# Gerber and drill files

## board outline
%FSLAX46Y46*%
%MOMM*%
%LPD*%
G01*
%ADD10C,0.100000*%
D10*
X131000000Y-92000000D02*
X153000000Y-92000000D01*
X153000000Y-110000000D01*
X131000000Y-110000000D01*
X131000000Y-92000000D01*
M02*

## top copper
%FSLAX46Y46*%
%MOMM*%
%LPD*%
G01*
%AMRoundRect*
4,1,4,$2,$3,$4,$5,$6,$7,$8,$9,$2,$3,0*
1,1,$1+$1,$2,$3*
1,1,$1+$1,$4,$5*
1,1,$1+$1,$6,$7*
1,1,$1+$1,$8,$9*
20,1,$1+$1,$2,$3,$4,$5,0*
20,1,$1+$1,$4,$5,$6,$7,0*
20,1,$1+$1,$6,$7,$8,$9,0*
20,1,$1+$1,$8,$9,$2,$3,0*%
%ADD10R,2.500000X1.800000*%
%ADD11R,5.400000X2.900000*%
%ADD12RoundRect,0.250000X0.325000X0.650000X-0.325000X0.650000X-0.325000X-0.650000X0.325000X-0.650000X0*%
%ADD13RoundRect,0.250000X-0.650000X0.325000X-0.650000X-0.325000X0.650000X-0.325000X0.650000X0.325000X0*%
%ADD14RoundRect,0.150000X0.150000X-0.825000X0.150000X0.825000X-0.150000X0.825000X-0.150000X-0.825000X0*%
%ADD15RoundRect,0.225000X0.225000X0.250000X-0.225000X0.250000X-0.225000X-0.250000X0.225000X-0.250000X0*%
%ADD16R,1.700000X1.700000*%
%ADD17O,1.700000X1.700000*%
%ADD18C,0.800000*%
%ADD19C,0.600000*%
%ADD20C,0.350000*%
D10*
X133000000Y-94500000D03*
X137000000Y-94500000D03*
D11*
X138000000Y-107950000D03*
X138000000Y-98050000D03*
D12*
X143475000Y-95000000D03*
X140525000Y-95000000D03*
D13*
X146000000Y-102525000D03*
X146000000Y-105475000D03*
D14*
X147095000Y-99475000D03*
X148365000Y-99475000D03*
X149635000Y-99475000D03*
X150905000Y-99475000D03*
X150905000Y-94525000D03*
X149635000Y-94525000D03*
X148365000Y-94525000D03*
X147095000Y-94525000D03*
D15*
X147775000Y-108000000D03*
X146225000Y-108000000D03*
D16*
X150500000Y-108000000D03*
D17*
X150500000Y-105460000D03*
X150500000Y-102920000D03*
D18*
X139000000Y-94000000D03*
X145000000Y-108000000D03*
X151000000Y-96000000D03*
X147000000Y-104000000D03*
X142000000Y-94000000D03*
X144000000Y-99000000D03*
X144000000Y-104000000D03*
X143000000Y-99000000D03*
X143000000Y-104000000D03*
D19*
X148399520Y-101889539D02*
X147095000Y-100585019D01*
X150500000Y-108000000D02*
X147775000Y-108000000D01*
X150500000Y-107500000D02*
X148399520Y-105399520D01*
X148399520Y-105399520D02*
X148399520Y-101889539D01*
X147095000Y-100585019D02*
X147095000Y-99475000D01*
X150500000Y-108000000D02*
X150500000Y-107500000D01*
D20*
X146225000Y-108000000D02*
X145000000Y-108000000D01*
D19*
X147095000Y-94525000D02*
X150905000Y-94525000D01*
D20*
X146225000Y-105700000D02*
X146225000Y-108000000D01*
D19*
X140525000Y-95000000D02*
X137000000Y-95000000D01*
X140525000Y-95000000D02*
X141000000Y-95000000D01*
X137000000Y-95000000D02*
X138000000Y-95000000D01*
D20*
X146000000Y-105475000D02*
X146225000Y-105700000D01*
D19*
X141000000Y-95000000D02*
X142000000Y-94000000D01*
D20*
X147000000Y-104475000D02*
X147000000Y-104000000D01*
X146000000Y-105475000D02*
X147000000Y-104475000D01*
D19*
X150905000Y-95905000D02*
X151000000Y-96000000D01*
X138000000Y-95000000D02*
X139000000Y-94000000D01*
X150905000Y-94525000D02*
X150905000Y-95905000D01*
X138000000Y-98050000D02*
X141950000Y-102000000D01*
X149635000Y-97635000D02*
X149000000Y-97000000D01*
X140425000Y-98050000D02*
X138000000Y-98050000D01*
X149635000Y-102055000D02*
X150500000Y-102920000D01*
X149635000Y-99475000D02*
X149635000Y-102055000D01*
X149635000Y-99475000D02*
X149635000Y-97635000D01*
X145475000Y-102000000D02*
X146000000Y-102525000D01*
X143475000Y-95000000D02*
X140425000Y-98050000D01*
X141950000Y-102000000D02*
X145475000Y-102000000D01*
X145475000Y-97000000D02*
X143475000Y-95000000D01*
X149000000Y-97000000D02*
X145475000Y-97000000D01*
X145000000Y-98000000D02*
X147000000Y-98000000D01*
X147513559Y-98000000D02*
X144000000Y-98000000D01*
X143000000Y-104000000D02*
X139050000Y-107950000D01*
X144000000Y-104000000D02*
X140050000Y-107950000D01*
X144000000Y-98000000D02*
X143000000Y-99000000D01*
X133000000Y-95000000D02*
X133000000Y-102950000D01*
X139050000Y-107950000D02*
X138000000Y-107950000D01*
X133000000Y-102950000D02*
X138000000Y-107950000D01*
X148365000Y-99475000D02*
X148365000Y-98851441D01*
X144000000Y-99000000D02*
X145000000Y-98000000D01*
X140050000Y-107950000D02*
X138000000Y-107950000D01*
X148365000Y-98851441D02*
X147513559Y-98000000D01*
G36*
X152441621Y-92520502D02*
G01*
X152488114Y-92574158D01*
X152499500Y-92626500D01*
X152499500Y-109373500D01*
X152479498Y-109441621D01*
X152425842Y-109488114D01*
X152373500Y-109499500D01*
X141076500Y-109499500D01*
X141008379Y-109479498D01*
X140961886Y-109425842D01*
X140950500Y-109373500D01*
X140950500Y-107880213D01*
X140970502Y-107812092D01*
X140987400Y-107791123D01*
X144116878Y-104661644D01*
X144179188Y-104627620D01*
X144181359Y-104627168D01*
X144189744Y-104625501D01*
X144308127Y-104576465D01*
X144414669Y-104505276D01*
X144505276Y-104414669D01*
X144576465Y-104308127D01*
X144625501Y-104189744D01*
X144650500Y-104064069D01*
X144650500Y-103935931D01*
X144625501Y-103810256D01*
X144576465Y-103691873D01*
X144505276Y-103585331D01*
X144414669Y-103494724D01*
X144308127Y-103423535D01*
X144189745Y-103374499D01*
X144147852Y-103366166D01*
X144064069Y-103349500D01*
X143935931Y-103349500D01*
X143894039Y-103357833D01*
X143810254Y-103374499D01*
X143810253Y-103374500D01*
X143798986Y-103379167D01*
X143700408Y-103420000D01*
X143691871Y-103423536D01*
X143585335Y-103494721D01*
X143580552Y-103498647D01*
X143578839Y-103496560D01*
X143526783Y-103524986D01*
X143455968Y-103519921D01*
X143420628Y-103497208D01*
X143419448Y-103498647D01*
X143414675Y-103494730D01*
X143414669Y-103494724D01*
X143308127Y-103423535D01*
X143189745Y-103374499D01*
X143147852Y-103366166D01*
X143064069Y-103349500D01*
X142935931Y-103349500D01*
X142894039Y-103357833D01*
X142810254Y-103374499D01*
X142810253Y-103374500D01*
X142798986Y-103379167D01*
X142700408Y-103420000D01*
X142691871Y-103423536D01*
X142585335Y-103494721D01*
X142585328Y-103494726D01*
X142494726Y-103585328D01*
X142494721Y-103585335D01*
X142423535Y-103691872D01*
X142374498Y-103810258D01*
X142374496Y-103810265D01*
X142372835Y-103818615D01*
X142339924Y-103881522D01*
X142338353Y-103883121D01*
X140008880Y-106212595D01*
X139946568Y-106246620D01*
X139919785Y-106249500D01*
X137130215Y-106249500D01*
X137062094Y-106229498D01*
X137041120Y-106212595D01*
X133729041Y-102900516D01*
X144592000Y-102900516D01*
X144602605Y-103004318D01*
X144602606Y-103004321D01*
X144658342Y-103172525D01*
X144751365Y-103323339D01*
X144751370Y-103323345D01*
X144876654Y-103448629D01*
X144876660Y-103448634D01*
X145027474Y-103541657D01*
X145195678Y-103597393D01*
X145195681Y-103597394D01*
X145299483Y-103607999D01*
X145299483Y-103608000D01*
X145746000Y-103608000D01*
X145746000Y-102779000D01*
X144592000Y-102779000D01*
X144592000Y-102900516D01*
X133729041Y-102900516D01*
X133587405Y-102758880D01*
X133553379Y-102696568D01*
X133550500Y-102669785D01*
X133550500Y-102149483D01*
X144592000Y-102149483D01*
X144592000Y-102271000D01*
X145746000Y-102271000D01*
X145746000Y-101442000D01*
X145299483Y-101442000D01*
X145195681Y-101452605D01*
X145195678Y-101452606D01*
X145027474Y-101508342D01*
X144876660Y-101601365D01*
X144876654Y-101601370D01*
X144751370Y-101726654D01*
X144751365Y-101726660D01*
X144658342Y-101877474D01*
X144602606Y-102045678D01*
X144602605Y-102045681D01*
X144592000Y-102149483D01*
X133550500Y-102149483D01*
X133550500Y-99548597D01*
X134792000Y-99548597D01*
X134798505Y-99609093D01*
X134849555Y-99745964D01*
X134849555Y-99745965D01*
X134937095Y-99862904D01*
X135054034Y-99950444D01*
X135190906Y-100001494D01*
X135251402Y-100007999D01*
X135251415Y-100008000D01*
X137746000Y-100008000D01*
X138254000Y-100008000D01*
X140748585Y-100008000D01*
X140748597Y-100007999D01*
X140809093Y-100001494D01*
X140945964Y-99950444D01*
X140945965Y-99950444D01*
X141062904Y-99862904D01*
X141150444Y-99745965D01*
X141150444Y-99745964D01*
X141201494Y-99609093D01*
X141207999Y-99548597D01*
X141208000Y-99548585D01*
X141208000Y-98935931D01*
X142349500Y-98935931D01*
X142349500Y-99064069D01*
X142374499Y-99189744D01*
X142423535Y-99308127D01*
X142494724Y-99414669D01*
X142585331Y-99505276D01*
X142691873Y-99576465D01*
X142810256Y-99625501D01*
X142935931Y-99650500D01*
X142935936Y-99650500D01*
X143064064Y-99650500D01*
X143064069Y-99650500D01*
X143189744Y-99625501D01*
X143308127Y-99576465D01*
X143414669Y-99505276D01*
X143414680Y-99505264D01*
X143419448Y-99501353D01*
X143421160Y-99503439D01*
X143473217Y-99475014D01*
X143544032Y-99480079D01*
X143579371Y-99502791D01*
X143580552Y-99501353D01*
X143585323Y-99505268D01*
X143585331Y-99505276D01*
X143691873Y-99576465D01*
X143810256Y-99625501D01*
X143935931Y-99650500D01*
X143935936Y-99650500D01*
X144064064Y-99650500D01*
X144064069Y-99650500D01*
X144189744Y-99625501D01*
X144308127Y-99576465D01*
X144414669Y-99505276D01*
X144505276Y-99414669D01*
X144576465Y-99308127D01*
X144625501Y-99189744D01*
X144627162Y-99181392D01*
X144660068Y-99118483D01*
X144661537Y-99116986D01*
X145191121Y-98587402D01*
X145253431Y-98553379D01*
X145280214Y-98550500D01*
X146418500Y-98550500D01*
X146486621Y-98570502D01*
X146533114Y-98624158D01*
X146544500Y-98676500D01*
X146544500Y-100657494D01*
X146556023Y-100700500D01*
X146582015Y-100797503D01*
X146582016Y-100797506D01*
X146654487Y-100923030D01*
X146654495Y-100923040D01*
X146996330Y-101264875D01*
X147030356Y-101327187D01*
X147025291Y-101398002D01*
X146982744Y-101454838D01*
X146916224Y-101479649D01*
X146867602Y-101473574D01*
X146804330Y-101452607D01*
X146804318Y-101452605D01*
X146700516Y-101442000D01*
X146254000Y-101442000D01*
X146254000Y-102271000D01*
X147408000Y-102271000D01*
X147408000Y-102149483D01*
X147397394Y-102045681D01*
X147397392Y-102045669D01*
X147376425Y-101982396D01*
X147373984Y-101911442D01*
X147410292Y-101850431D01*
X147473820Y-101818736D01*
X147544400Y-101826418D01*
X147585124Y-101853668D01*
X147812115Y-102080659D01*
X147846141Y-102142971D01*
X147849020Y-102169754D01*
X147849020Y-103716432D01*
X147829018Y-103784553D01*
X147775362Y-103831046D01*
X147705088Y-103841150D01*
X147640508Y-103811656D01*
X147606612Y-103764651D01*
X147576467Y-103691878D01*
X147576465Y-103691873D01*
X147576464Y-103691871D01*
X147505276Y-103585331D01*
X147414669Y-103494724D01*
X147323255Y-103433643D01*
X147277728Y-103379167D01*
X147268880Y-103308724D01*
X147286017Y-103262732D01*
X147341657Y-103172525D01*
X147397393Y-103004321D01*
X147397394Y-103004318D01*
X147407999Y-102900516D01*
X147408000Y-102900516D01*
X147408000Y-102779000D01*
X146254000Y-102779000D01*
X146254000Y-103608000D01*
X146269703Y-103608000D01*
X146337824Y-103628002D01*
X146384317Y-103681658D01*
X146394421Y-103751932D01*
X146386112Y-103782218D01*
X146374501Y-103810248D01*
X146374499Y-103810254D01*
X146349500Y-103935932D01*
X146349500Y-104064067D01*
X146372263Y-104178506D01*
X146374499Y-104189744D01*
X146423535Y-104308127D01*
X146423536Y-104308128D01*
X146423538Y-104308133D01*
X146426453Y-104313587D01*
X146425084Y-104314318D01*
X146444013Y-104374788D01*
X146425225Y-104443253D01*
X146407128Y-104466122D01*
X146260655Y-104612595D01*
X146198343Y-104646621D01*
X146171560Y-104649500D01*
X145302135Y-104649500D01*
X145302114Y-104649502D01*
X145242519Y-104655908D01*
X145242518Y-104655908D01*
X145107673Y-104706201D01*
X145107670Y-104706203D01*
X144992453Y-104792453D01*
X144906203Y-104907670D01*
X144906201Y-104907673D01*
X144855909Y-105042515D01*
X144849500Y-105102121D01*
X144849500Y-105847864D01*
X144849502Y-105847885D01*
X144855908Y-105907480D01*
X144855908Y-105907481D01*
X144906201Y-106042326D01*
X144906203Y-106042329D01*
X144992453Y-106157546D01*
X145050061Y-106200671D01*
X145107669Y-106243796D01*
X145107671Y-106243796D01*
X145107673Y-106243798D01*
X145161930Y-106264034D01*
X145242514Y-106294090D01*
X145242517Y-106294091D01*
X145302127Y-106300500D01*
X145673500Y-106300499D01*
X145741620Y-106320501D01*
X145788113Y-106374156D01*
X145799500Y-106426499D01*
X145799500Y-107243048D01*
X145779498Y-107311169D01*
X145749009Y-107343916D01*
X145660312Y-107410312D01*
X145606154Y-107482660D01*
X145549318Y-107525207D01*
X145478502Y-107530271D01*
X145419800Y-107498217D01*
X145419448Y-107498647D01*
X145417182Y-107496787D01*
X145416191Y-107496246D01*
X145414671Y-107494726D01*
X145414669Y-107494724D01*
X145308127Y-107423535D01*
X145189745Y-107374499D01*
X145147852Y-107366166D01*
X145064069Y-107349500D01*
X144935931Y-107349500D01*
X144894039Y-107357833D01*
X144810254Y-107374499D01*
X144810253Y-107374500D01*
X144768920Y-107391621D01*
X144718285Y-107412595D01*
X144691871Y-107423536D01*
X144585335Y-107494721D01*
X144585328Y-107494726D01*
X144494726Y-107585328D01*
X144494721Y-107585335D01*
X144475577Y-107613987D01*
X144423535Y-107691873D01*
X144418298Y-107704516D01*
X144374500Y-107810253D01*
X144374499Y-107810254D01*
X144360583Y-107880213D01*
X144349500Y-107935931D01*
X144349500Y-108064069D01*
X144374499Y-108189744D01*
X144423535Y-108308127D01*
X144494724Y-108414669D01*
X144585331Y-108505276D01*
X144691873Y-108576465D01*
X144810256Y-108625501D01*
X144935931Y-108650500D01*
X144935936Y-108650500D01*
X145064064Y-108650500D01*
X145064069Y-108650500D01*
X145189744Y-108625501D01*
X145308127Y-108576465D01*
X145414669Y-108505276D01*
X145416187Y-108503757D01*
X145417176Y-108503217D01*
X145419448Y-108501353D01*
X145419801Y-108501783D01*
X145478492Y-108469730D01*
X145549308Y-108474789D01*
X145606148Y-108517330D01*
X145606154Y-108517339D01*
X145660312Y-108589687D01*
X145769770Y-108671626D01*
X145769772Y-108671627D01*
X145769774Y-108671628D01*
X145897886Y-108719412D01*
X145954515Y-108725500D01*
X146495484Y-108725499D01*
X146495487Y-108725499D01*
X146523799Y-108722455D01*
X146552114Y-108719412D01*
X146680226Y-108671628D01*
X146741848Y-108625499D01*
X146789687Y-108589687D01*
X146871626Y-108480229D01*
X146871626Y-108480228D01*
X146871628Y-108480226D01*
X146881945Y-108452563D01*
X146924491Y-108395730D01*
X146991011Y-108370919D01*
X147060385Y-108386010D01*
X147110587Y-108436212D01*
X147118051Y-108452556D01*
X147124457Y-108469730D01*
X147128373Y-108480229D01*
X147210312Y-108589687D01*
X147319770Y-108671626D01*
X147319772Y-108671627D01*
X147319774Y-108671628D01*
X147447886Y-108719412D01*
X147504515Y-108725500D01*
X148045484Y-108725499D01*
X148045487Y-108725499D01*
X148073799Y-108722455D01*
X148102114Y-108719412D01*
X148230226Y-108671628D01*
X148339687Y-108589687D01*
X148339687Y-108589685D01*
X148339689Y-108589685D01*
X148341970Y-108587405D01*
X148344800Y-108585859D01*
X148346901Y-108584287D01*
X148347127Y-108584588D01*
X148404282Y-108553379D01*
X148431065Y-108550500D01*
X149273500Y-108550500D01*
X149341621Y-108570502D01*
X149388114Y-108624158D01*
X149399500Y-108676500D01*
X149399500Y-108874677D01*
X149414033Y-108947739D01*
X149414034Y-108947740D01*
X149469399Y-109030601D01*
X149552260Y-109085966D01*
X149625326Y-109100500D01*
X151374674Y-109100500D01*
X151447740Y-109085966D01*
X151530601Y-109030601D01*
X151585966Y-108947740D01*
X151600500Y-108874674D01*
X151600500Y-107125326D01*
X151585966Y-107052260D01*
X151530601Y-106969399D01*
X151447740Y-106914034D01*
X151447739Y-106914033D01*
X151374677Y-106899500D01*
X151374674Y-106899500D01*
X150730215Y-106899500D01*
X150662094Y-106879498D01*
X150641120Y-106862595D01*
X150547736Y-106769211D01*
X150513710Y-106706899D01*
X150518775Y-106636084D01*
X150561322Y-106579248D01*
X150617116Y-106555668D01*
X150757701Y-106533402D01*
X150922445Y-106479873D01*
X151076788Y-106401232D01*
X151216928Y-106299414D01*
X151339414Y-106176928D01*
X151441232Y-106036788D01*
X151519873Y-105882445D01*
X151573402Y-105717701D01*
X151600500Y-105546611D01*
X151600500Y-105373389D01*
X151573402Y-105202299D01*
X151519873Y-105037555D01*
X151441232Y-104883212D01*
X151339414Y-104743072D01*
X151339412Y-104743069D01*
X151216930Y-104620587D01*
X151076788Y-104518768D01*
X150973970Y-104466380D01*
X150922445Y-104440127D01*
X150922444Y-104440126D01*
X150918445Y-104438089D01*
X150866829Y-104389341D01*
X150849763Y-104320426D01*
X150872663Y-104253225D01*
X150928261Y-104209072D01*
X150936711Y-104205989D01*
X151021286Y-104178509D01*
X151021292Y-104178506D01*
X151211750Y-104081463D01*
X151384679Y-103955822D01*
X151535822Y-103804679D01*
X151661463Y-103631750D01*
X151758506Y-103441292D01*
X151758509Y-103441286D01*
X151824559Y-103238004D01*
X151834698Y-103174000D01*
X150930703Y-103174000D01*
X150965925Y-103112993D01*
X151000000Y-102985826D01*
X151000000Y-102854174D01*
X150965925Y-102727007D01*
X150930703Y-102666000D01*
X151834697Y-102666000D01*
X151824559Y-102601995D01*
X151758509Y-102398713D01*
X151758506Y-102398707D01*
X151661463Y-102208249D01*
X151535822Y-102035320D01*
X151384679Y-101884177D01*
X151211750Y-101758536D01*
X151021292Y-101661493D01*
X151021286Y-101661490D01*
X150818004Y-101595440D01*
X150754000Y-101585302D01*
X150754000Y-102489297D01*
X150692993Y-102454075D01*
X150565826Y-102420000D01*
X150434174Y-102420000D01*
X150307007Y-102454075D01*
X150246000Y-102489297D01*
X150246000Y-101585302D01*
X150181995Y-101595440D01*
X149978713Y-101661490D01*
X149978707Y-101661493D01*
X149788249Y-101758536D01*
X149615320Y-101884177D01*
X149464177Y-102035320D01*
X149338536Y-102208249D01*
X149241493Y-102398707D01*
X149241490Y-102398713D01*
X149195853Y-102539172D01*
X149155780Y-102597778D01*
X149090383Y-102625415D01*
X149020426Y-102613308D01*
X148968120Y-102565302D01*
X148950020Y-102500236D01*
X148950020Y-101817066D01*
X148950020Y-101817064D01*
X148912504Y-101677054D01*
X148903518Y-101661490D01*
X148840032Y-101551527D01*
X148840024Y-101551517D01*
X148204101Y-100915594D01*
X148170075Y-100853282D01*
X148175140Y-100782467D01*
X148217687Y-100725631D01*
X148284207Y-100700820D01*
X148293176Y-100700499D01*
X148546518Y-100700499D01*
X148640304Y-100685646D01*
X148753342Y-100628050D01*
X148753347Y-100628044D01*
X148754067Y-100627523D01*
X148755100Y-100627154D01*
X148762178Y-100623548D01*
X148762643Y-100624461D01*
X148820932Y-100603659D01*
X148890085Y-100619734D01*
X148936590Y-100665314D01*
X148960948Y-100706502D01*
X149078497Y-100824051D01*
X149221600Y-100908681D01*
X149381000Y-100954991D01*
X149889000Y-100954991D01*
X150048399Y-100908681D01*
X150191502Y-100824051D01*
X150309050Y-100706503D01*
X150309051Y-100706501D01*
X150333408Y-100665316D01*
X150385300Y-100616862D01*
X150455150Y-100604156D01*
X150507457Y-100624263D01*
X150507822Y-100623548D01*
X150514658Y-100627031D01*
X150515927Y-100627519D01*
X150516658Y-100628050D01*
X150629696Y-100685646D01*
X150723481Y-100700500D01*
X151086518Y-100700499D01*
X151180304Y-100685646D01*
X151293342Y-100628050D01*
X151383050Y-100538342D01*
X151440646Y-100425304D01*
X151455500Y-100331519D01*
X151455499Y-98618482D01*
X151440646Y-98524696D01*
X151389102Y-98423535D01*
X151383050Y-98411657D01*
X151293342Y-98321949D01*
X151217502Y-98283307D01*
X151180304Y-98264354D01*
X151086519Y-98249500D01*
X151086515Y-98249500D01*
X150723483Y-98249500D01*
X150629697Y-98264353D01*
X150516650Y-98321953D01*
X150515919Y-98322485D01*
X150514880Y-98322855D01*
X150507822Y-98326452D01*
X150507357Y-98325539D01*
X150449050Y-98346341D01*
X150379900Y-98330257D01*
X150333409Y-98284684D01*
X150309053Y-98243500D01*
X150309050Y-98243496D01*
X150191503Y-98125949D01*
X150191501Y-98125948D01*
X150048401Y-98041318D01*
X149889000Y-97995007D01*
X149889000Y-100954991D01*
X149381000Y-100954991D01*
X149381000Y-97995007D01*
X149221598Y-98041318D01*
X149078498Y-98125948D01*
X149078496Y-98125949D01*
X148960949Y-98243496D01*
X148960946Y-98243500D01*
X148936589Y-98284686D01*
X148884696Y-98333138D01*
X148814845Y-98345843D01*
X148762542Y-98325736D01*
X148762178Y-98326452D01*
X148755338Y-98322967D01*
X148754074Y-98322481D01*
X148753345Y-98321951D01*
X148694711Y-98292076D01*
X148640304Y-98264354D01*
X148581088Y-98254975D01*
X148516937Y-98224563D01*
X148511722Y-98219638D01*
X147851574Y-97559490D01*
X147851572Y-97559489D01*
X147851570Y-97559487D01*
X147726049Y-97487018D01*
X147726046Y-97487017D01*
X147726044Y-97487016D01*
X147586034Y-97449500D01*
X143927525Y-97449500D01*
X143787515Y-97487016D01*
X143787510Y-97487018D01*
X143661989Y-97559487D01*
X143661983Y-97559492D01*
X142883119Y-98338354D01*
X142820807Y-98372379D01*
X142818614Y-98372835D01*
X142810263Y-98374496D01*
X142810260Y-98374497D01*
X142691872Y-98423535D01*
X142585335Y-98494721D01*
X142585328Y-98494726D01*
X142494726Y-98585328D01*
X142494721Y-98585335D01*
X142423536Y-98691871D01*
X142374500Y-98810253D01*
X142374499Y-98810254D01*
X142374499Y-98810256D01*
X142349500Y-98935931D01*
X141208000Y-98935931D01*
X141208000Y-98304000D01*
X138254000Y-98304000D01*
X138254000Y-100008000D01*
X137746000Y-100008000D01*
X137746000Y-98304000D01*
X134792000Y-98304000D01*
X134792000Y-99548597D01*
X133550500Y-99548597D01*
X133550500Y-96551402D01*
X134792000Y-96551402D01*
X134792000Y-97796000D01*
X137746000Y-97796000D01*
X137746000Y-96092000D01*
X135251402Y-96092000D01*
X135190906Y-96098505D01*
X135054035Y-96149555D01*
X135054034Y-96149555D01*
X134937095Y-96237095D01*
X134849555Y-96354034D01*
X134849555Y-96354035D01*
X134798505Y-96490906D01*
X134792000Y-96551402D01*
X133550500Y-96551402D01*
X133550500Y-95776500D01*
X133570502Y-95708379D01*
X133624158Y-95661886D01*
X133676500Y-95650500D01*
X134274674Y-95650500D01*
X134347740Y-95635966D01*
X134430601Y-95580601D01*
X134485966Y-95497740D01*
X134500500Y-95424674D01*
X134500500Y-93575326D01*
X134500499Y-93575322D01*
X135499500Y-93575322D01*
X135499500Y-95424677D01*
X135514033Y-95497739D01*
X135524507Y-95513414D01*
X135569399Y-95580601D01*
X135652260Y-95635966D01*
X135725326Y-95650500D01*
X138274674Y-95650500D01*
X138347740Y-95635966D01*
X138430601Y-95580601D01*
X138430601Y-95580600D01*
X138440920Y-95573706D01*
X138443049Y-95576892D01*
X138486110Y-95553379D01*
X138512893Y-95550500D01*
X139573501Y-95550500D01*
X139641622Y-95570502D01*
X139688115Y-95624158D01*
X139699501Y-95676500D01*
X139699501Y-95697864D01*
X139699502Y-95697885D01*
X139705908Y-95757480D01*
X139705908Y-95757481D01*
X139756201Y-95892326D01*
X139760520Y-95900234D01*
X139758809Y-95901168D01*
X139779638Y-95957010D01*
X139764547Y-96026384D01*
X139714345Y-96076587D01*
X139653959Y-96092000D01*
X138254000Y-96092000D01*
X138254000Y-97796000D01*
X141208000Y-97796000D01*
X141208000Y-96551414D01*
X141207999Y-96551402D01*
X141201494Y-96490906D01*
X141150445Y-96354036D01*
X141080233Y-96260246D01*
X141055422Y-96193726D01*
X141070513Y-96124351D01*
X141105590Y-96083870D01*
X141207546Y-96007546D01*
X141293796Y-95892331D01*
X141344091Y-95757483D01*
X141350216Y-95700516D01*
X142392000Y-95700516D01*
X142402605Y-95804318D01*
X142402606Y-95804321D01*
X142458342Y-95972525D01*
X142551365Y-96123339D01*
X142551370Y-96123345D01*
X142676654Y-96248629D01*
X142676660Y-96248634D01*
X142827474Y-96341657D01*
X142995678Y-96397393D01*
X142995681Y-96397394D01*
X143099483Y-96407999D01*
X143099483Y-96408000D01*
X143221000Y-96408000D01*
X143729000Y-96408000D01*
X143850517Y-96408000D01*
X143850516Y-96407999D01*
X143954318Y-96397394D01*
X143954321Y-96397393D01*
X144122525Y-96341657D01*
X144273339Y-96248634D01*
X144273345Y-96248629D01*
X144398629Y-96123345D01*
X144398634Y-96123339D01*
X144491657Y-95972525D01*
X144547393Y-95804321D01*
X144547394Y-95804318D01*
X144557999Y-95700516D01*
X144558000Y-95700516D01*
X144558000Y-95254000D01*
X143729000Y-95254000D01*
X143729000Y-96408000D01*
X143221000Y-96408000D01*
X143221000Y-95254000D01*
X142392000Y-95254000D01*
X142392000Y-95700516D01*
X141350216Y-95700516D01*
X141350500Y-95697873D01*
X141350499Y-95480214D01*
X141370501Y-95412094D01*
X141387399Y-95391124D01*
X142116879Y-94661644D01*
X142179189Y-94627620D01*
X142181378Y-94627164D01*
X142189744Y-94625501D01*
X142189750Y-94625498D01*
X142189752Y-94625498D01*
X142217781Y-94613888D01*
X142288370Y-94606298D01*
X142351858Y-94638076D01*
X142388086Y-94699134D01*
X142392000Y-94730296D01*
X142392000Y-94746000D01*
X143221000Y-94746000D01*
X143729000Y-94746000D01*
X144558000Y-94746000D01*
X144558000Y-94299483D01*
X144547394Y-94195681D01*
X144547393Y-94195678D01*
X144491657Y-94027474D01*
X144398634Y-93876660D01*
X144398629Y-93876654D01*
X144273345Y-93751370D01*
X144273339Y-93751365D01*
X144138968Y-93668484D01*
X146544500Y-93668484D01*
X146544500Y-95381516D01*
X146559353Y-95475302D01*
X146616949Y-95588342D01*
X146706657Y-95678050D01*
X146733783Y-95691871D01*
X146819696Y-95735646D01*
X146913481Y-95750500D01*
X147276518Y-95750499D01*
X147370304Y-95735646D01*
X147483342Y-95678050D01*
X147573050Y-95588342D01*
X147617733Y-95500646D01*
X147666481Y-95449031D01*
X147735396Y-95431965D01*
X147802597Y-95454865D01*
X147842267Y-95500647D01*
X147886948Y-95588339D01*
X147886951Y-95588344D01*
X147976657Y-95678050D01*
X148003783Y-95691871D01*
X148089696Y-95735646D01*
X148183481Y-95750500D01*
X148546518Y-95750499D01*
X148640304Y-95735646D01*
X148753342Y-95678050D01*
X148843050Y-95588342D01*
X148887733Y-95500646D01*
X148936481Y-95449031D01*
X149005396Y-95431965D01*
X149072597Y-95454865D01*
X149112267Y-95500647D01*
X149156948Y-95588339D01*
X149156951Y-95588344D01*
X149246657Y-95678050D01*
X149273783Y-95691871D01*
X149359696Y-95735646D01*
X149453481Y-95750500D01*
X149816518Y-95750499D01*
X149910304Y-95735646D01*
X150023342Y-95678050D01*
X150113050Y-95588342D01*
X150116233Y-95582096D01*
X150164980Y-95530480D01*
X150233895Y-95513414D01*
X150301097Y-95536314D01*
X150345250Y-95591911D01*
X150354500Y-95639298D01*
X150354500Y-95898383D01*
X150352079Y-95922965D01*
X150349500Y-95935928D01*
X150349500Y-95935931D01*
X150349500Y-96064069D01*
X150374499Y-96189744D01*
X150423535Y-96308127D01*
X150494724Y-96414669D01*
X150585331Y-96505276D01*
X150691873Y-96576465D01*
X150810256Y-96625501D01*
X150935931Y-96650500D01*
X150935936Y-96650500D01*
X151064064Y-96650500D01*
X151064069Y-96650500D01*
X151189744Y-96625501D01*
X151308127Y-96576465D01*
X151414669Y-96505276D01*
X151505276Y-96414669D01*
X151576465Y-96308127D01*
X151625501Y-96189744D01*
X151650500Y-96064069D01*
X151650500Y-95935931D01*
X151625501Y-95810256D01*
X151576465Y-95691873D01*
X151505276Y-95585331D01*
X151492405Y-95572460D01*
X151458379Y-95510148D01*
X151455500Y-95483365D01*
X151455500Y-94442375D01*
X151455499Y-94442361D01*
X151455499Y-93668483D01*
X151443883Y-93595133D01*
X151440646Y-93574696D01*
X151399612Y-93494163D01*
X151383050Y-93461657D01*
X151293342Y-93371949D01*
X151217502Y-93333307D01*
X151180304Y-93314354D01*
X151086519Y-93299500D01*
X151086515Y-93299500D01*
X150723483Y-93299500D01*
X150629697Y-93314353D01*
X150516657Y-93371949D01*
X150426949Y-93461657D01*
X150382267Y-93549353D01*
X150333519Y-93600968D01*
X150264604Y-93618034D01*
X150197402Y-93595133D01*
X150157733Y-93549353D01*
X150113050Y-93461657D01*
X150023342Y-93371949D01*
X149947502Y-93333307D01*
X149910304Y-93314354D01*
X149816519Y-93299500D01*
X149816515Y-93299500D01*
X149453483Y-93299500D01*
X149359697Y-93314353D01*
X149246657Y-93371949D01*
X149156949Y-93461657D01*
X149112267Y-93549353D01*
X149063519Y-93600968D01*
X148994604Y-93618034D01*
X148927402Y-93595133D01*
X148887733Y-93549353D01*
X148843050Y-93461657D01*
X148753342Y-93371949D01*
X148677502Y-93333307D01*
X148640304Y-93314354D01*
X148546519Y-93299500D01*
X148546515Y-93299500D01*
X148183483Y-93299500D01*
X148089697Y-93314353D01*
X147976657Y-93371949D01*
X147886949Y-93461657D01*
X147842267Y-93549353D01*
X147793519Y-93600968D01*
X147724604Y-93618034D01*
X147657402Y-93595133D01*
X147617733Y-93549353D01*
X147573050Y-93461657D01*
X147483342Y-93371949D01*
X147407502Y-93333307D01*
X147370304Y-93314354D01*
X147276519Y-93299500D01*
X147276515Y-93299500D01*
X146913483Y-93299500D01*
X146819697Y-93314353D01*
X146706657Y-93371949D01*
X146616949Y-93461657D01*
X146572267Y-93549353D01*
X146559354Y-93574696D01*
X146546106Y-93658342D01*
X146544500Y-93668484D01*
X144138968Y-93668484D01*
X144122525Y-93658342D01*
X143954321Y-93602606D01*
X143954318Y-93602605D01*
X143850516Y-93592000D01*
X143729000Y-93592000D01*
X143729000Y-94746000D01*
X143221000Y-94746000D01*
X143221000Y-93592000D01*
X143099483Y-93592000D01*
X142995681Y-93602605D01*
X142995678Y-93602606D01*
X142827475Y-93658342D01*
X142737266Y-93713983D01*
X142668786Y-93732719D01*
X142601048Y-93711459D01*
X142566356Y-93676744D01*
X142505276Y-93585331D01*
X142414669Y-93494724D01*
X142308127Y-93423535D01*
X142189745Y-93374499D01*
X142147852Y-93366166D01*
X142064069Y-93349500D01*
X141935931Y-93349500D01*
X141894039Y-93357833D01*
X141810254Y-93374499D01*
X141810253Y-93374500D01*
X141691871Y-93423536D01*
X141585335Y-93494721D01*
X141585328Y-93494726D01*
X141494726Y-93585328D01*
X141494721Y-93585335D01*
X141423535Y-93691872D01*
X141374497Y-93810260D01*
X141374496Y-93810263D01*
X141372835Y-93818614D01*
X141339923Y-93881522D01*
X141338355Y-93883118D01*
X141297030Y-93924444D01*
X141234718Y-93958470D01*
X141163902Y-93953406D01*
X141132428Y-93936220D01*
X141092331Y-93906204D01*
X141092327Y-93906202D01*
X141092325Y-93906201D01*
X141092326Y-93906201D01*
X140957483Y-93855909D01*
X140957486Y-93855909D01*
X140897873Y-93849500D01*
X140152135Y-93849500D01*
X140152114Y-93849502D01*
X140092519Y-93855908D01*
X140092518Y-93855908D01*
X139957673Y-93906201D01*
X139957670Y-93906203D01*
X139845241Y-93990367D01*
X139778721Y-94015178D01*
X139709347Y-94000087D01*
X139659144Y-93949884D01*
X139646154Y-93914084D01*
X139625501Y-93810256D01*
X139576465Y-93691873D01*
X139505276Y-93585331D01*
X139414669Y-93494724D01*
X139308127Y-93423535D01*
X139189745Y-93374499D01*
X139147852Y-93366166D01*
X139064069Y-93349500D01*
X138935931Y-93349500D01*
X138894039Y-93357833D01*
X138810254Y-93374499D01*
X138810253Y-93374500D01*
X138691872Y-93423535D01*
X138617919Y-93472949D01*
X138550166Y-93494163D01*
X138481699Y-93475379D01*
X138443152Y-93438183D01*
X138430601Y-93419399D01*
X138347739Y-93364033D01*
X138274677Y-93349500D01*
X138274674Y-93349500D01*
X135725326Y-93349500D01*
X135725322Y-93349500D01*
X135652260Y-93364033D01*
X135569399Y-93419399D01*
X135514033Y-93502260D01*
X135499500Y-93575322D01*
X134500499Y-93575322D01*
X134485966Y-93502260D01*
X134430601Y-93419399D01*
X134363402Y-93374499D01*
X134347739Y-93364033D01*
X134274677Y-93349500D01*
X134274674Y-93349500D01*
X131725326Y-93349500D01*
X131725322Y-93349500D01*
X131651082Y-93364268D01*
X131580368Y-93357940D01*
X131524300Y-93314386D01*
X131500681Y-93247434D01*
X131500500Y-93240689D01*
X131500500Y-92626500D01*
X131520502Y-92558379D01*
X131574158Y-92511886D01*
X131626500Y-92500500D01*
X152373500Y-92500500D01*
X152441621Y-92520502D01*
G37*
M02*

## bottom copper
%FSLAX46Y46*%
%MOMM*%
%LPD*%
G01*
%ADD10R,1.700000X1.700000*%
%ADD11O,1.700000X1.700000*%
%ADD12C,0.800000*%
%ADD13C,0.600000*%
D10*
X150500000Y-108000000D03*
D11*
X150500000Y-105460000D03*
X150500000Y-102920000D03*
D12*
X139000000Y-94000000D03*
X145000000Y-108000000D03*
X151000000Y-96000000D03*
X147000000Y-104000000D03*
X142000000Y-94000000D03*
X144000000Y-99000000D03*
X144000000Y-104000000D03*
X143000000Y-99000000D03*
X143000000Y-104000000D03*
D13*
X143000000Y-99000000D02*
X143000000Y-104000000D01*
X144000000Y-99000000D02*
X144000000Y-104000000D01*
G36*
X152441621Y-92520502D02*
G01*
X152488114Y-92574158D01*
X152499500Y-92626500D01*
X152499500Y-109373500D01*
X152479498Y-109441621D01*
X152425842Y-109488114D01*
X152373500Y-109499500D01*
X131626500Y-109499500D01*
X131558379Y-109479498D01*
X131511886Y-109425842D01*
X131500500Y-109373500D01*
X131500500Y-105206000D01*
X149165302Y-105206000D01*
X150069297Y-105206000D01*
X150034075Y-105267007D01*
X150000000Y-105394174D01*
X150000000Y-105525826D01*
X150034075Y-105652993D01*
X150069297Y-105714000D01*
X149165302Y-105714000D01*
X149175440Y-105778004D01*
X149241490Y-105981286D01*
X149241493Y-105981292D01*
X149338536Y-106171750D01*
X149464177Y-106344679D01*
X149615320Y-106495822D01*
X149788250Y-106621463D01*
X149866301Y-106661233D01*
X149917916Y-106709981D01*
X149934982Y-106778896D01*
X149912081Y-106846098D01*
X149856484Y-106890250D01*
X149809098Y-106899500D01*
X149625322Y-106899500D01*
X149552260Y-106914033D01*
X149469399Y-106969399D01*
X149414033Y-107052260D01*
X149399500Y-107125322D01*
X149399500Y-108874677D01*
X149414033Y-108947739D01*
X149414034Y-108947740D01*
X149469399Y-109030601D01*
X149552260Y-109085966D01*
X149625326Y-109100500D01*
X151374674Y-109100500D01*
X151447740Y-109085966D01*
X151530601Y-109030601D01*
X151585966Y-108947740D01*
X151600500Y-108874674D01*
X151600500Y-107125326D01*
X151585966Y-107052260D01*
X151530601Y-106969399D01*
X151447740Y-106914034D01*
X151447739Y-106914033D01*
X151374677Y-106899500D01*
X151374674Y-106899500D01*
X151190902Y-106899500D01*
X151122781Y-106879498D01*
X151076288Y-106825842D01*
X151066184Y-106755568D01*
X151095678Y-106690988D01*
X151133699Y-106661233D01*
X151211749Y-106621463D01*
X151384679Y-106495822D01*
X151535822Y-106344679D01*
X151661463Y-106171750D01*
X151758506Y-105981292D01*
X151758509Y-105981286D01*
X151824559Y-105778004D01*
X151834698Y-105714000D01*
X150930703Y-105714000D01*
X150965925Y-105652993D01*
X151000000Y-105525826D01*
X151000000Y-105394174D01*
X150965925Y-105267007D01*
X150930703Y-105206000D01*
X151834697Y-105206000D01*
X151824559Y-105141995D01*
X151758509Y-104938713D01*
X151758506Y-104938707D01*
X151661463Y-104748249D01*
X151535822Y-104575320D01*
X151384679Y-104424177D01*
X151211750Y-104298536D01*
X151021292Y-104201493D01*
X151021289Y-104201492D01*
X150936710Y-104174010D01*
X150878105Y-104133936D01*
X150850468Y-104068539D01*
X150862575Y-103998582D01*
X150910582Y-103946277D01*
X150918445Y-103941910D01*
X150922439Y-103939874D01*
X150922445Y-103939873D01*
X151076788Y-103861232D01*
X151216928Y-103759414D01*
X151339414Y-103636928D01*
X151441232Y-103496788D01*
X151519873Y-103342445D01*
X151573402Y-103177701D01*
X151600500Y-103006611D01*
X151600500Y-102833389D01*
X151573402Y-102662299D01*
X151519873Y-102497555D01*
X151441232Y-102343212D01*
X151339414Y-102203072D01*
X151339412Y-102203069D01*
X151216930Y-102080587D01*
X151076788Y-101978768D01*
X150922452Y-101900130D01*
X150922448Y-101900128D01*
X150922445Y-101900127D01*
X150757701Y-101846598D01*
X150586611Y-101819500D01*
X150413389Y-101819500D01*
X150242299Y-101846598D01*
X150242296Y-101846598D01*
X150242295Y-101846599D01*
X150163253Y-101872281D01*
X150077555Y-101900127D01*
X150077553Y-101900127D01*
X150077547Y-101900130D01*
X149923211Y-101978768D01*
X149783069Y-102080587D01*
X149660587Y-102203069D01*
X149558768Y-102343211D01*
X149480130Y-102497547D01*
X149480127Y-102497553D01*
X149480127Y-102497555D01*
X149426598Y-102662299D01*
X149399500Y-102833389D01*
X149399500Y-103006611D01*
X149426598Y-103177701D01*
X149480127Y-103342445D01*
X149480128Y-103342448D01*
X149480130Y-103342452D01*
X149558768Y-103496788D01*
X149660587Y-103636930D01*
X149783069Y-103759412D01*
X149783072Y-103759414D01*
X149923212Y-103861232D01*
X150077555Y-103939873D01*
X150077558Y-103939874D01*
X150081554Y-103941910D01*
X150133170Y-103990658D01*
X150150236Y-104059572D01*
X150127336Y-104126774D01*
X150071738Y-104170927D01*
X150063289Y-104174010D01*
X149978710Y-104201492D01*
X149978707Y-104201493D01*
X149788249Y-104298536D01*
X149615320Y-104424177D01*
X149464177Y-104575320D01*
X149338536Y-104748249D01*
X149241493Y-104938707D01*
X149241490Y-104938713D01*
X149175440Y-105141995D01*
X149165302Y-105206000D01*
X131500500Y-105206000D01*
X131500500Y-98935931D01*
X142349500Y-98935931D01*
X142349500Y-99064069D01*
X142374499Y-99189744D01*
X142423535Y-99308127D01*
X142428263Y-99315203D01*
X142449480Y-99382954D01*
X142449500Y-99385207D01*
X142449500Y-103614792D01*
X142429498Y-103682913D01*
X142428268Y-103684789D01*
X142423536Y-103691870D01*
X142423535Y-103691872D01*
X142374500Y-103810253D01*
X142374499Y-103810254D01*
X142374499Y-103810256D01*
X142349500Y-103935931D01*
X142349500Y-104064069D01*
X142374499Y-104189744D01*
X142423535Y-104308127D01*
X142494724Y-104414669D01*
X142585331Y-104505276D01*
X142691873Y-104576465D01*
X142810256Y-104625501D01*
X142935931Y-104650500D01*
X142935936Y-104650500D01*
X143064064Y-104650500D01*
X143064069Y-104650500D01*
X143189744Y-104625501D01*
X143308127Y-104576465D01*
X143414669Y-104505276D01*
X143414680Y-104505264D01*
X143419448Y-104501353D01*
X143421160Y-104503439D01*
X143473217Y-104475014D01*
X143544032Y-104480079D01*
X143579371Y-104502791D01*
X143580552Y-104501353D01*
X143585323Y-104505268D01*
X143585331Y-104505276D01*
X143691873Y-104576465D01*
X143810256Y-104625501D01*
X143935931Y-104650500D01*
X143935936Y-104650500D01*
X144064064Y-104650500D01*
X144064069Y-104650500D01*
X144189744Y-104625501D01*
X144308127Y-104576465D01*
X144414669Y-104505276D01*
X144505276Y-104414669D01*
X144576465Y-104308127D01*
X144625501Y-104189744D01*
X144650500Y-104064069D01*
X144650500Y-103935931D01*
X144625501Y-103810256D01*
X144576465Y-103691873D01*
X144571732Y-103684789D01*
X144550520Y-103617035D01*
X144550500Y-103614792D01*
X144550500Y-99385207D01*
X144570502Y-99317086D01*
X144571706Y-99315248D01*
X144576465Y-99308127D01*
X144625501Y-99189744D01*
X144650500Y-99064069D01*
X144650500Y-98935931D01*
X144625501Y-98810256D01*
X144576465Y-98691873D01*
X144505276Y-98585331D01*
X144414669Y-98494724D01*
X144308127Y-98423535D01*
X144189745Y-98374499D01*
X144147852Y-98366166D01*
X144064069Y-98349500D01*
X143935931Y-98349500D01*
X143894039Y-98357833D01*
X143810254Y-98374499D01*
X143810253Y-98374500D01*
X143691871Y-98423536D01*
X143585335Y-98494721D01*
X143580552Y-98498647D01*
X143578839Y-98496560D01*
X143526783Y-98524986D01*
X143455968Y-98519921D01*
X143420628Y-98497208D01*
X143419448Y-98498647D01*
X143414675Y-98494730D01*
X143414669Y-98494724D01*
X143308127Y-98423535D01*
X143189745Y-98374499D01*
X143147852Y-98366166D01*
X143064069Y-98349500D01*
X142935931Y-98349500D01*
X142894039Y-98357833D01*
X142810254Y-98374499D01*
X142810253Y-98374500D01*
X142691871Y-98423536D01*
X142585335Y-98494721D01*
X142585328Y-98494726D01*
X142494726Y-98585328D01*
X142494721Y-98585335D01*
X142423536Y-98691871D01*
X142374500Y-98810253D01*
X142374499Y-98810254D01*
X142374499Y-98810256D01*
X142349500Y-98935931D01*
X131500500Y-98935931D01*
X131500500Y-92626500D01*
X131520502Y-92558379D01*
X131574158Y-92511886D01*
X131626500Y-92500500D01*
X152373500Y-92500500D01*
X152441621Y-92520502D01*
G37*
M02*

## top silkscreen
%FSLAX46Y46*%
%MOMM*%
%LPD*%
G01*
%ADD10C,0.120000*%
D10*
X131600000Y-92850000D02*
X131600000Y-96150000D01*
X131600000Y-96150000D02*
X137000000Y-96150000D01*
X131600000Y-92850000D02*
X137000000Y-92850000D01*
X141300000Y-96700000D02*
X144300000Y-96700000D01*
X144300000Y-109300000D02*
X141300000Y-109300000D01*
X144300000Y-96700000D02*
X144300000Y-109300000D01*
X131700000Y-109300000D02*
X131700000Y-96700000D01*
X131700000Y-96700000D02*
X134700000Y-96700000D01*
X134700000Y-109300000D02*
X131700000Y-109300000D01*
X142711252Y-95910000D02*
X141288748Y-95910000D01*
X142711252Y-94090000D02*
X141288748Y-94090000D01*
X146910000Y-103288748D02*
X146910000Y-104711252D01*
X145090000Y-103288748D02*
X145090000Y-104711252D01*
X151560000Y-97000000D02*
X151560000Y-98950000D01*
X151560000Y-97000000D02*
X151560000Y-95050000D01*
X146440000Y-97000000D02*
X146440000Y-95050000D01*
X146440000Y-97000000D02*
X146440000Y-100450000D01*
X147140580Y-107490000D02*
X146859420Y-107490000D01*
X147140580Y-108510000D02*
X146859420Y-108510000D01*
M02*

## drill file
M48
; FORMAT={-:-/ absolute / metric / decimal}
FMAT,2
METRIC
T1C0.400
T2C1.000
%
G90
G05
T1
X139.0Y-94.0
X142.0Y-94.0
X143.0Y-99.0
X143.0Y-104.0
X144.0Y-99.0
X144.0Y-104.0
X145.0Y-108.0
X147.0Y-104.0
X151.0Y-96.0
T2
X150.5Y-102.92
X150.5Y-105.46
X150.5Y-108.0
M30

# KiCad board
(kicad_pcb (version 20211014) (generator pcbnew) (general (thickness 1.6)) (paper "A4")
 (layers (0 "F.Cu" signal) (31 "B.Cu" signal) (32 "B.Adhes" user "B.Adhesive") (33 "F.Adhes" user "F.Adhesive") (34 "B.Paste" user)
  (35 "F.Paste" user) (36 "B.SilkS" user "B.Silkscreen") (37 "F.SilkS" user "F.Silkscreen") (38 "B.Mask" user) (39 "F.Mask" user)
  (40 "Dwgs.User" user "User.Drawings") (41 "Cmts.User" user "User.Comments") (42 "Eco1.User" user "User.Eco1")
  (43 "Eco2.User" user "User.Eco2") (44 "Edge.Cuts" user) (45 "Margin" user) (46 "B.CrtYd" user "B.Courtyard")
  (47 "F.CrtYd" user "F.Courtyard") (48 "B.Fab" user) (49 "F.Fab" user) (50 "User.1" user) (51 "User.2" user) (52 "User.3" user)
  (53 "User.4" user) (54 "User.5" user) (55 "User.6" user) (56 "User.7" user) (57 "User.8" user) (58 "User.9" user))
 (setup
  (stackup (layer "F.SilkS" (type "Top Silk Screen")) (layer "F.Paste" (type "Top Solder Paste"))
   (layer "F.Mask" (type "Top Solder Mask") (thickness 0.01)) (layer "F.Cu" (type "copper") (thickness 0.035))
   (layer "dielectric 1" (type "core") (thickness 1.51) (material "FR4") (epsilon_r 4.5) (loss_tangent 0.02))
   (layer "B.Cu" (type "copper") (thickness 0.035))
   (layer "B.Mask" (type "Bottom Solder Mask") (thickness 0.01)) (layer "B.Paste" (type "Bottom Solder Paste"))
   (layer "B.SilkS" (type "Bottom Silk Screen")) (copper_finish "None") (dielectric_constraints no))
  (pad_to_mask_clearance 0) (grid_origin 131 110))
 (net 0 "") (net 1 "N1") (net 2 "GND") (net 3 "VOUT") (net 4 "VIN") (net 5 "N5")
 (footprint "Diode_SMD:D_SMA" (layer "F.Cu") (at 135 94.5)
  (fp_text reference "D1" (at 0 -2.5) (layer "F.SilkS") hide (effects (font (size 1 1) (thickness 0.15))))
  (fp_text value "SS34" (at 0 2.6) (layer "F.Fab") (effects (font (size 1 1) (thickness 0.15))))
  (fp_line (start -3.4 -1.65) (end -3.4 1.65) (layer "F.SilkS") (width 0.12))
  (fp_line (start -3.4 1.65) (end 2 1.65) (layer "F.SilkS") (width 0.12))
  (fp_line (start -3.4 -1.65) (end 2 -1.65) (layer "F.SilkS") (width 0.12))
  (pad "1" smd rect locked (at -2 0) (size 2.5 1.8) (layers "F.Cu" "F.Paste" "F.Mask") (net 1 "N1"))
  (pad "2" smd rect locked (at 2 0) (size 2.5 1.8) (layers "F.Cu" "F.Paste" "F.Mask") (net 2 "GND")))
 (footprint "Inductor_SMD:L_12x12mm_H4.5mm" (layer "F.Cu") (at 138 103 90)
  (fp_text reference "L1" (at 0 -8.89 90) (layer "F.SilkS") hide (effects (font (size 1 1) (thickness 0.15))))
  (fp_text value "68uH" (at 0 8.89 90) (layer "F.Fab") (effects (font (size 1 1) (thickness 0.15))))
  (fp_line (start 6.3 3.3) (end 6.3 6.3) (layer "F.SilkS") (width 0.12))
  (fp_line (start -6.3 6.3) (end -6.3 3.3) (layer "F.SilkS") (width 0.12))
  (fp_line (start 6.3 6.3) (end -6.3 6.3) (layer "F.SilkS") (width 0.12))
  (fp_line (start -6.3 -6.3) (end 6.3 -6.3) (layer "F.SilkS") (width 0.12))
  (fp_line (start 6.3 -6.3) (end 6.3 -3.3) (layer "F.SilkS") (width 0.12))
  (fp_line (start -6.3 -3.3) (end -6.3 -6.3) (layer "F.SilkS") (width 0.12))
  (pad "1" smd rect locked (at -4.95 0 90) (size 2.9 5.4) (layers "F.Cu" "F.Paste" "F.Mask") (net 1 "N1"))
  (pad "2" smd rect locked (at 4.95 0 90) (size 2.9 5.4) (layers "F.Cu" "F.Paste" "F.Mask") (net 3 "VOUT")))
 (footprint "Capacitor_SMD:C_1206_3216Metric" (layer "F.Cu") (at 142 95 180)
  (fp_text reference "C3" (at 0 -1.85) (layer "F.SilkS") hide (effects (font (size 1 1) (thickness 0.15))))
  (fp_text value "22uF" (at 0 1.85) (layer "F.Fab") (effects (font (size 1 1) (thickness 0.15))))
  (fp_line (start -0.711252 -0.91) (end 0.711252 -0.91) (layer "F.SilkS") (width 0.12))
  (fp_line (start -0.711252 0.91) (end 0.711252 0.91) (layer "F.SilkS") (width 0.12))
  (pad "1" smd roundrect locked (at -1.475 0 180) (size 1.15 1.8) (layers "F.Cu" "F.Paste" "F.Mask") (roundrect_rratio 0.217391)
   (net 3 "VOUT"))
  (pad "2" smd roundrect locked (at 1.475 0 180) (size 1.15 1.8) (layers "F.Cu" "F.Paste" "F.Mask") (roundrect_rratio 0.217391)
   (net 2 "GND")))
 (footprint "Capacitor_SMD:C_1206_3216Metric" (layer "F.Cu") (at 146 104 -90)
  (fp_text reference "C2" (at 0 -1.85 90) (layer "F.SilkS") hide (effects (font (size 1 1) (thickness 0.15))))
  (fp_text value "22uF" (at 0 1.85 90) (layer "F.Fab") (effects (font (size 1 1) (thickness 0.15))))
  (fp_line (start -0.711252 -0.91) (end 0.711252 -0.91) (layer "F.SilkS") (width 0.12))
  (fp_line (start -0.711252 0.91) (end 0.711252 0.91) (layer "F.SilkS") (width 0.12))
  (pad "1" smd roundrect locked (at -1.475 0 270) (size 1.15 1.8) (layers "F.Cu" "F.Paste" "F.Mask") (roundrect_rratio 0.217391)
   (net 3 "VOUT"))
  (pad "2" smd roundrect locked (at 1.475 0 270) (size 1.15 1.8) (layers "F.Cu" "F.Paste" "F.Mask") (roundrect_rratio 0.217391)
   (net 2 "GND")))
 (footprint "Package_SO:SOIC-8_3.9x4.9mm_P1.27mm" (layer "F.Cu") (at 149 97 90)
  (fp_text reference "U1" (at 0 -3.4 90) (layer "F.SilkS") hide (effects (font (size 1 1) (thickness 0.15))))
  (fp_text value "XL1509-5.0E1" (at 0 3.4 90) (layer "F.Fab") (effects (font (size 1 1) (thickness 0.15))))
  (fp_line (start 0 2.56) (end -1.95 2.56) (layer "F.SilkS") (width 0.12))
  (fp_line (start 0 2.56) (end 1.95 2.56) (layer "F.SilkS") (width 0.12))
  (fp_line (start 0 -2.56) (end 1.95 -2.56) (layer "F.SilkS") (width 0.12))
  (fp_line (start 0 -2.56) (end -3.45 -2.56) (layer "F.SilkS") (width 0.12))
  (pad "1" smd roundrect locked (at -2.475 -1.905 90) (size 1.95 0.6) (layers "F.Cu" "F.Paste" "F.Mask") (roundrect_rratio 0.25)
   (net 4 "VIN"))
  (pad "2" smd roundrect locked (at -2.475 -0.635 90) (size 1.95 0.6) (layers "F.Cu" "F.Paste" "F.Mask") (roundrect_rratio 0.25)
   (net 1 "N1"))
  (pad "3" smd roundrect locked (at -2.475 0.635 90) (size 1.95 0.6) (layers "F.Cu" "F.Paste" "F.Mask") (roundrect_rratio 0.25)
   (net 3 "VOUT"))
  (pad "4" smd roundrect locked (at -2.475 1.905 90) (size 1.95 0.6) (layers "F.Cu" "F.Paste" "F.Mask") (roundrect_rratio 0.25) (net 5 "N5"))
  (pad "5" smd roundrect locked (at 2.475 1.905 90) (size 1.95 0.6) (layers "F.Cu" "F.Paste" "F.Mask") (roundrect_rratio 0.25) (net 2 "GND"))
  (pad "6" smd roundrect locked (at 2.475 0.635 90) (size 1.95 0.6) (layers "F.Cu" "F.Paste" "F.Mask") (roundrect_rratio 0.25) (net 2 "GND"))
  (pad "7" smd roundrect locked (at 2.475 -0.635 90) (size 1.95 0.6) (layers "F.Cu" "F.Paste" "F.Mask") (roundrect_rratio 0.25)
   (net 2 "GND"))
  (pad "8" smd roundrect locked (at 2.475 -1.905 90) (size 1.95 0.6) (layers "F.Cu" "F.Paste" "F.Mask") (roundrect_rratio 0.25)
   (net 2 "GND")))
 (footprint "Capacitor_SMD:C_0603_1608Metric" (layer "F.Cu") (at 147 108 180)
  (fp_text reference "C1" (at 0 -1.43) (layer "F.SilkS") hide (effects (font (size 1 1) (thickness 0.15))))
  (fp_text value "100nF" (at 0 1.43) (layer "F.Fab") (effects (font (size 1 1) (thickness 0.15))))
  (fp_line (start -0.14058 0.51) (end 0.14058 0.51) (layer "F.SilkS") (width 0.12))
  (fp_line (start -0.14058 -0.51) (end 0.14058 -0.51) (layer "F.SilkS") (width 0.12))
  (pad "1" smd roundrect locked (at -0.775 0 180) (size 0.9 0.95) (layers "F.Cu" "F.Paste" "F.Mask") (roundrect_rratio 0.25) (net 4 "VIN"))
  (pad "2" smd roundrect locked (at 0.775 0 180) (size 0.9 0.95) (layers "F.Cu" "F.Paste" "F.Mask") (roundrect_rratio 0.25) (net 2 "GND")))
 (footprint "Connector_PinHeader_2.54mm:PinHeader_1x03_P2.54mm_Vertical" (layer "B.Cu") (at 150.5 108)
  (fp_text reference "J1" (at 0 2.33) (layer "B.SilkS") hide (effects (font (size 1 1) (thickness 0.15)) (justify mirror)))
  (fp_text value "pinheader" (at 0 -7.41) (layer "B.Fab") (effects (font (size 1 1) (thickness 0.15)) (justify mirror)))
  (pad "1" thru_hole rect locked (at 0 0) (size 1.7 1.7) (drill 1) (layers *.Cu *.Mask) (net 4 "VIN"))
  (pad "2" thru_hole oval locked (at 0 -2.54) (size 1.7 1.7) (drill 1) (layers *.Cu *.Mask) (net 2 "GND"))
  (pad "3" thru_hole oval locked (at 0 -5.08) (size 1.7 1.7) (drill 1) (layers *.Cu *.Mask) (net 3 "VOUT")))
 (gr_rect (start 153 92) (end 131 110) (layer "Edge.Cuts") (width 0.1) (fill none))
 (segment (start 148.39952 101.889539) (end 147.095 100.585019) (width 0.6) (layer "F.Cu") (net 4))
 (segment (start 150.5 108) (end 147.775 108) (width 0.6) (layer "F.Cu") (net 4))
 (segment (start 150.5 107.5) (end 148.39952 105.39952) (width 0.6) (layer "F.Cu") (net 4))
 (segment (start 148.39952 105.39952) (end 148.39952 101.889539) (width 0.6) (layer "F.Cu") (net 4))
 (segment (start 147.095 100.585019) (end 147.095 99.475) (width 0.6) (layer "F.Cu") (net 4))
 (segment (start 150.5 108) (end 150.5 107.5) (width 0.6) (layer "F.Cu") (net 4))
 (segment (start 146.225 108) (end 145 108) (width 0.35) (layer "F.Cu") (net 2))
 (segment (start 147.095 94.525) (end 150.905 94.525) (width 0.6) (layer "F.Cu") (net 2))
 (segment (start 146.225 105.7) (end 146.225 108) (width 0.35) (layer "F.Cu") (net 2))
 (segment (start 140.525 95) (end 137 95) (width 0.6) (layer "F.Cu") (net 2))
 (segment (start 140.525 95) (end 141 95) (width 0.6) (layer "F.Cu") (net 2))
 (segment (start 137 95) (end 138 95) (width 0.6) (layer "F.Cu") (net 2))
 (segment (start 146 105.475) (end 146.225 105.7) (width 0.35) (layer "F.Cu") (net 2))
 (segment (start 141 95) (end 142 94) (width 0.6) (layer "F.Cu") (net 2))
 (segment (start 147 104.475) (end 147 104) (width 0.35) (layer "F.Cu") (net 2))
 (segment (start 146 105.475) (end 147 104.475) (width 0.35) (layer "F.Cu") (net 2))
 (segment (start 150.905 95.905) (end 151 96) (width 0.6) (layer "F.Cu") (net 2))
 (segment (start 138 95) (end 139 94) (width 0.6) (layer "F.Cu") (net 2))
 (segment (start 150.905 94.525) (end 150.905 95.905) (width 0.6) (layer "F.Cu") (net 2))
 (via (at 139 94) (size 0.8) (drill 0.4) (layers "F.Cu" "B.Cu") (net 2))
 (via (at 145 108) (size 0.8) (drill 0.4) (layers "F.Cu" "B.Cu") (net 2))
 (via (at 151 96) (size 0.8) (drill 0.4) (layers "F.Cu" "B.Cu") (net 2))
 (via (at 147 104) (size 0.8) (drill 0.4) (layers "F.Cu" "B.Cu") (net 2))
 (via (at 142 94) (size 0.8) (drill 0.4) (layers "F.Cu" "B.Cu") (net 2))
 (segment (start 138 98.05) (end 141.95 102) (width 0.6) (layer "F.Cu") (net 3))
 (segment (start 149.635 97.635) (end 149 97) (width 0.6) (layer "F.Cu") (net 3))
 (segment (start 140.425 98.05) (end 138 98.05) (width 0.6) (layer "F.Cu") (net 3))
 (segment (start 149.635 102.055) (end 150.5 102.92) (width 0.6) (layer "F.Cu") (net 3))
 (segment (start 149.635 99.475) (end 149.635 102.055) (width 0.6) (layer "F.Cu") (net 3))
 (segment (start 149.635 99.475) (end 149.635 97.635) (width 0.6) (layer "F.Cu") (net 3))
 (segment (start 145.475 102) (end 146 102.525) (width 0.6) (layer "F.Cu") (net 3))
 (segment (start 143.475 95) (end 140.425 98.05) (width 0.6) (layer "F.Cu") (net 3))
 (segment (start 141.95 102) (end 145.475 102) (width 0.6) (layer "F.Cu") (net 3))
 (segment (start 145.475 97) (end 143.475 95) (width 0.6) (layer "F.Cu") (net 3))
 (segment (start 149 97) (end 145.475 97) (width 0.6) (layer "F.Cu") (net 3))
 (segment (start 145 98) (end 147 98) (width 0.6) (layer "F.Cu") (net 1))
 (segment (start 147.513559 98) (end 144 98) (width 0.6) (layer "F.Cu") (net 1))
 (segment (start 143 104) (end 139.05 107.95) (width 0.6) (layer "F.Cu") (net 1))
 (segment (start 144 104) (end 140.05 107.95) (width 0.6) (layer "F.Cu") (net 1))
 (segment (start 144 98) (end 143 99) (width 0.6) (layer "F.Cu") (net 1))
 (segment (start 133 95) (end 133 102.95) (width 0.6) (layer "F.Cu") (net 1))
 (segment (start 139.05 107.95) (end 138 107.95) (width 0.6) (layer "F.Cu") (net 1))
 (segment (start 133 102.95) (end 138 107.95) (width 0.6) (layer "F.Cu") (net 1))
 (segment (start 148.365 99.475) (end 148.365 98.851441) (width 0.6) (layer "F.Cu") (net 1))
 (segment (start 144 99) (end 145 98) (width 0.6) (layer "F.Cu") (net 1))
 (segment (start 140.05 107.95) (end 138 107.95) (width 0.6) (layer "F.Cu") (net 1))
 (segment (start 148.365 98.851441) (end 147.513559 98) (width 0.6) (layer "F.Cu") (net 1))
 (via (at 144 99) (size 0.8) (drill 0.4) (layers "F.Cu" "B.Cu") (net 1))
 (via (at 144 104) (size 0.8) (drill 0.4) (layers "F.Cu" "B.Cu") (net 1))
 (via (at 143 99) (size 0.8) (drill 0.4) (layers "F.Cu" "B.Cu") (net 1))
 (via (at 143 104) (size 0.8) (drill 0.4) (layers "F.Cu" "B.Cu") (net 1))
 (segment (start 143 99) (end 143 104) (width 0.6) (layer "B.Cu") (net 1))
 (segment (start 144 99) (end 144 104) (width 0.6) (layer "B.Cu") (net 1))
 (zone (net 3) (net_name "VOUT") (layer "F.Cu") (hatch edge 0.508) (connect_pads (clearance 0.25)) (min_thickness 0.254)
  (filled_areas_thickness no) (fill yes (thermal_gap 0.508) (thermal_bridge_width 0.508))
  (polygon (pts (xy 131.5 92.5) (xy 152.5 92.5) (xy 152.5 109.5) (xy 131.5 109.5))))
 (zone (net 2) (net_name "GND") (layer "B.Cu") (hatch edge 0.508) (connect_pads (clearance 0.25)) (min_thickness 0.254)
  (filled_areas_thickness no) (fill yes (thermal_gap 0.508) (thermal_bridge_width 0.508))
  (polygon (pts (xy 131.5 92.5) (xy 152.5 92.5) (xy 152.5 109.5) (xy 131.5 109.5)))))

